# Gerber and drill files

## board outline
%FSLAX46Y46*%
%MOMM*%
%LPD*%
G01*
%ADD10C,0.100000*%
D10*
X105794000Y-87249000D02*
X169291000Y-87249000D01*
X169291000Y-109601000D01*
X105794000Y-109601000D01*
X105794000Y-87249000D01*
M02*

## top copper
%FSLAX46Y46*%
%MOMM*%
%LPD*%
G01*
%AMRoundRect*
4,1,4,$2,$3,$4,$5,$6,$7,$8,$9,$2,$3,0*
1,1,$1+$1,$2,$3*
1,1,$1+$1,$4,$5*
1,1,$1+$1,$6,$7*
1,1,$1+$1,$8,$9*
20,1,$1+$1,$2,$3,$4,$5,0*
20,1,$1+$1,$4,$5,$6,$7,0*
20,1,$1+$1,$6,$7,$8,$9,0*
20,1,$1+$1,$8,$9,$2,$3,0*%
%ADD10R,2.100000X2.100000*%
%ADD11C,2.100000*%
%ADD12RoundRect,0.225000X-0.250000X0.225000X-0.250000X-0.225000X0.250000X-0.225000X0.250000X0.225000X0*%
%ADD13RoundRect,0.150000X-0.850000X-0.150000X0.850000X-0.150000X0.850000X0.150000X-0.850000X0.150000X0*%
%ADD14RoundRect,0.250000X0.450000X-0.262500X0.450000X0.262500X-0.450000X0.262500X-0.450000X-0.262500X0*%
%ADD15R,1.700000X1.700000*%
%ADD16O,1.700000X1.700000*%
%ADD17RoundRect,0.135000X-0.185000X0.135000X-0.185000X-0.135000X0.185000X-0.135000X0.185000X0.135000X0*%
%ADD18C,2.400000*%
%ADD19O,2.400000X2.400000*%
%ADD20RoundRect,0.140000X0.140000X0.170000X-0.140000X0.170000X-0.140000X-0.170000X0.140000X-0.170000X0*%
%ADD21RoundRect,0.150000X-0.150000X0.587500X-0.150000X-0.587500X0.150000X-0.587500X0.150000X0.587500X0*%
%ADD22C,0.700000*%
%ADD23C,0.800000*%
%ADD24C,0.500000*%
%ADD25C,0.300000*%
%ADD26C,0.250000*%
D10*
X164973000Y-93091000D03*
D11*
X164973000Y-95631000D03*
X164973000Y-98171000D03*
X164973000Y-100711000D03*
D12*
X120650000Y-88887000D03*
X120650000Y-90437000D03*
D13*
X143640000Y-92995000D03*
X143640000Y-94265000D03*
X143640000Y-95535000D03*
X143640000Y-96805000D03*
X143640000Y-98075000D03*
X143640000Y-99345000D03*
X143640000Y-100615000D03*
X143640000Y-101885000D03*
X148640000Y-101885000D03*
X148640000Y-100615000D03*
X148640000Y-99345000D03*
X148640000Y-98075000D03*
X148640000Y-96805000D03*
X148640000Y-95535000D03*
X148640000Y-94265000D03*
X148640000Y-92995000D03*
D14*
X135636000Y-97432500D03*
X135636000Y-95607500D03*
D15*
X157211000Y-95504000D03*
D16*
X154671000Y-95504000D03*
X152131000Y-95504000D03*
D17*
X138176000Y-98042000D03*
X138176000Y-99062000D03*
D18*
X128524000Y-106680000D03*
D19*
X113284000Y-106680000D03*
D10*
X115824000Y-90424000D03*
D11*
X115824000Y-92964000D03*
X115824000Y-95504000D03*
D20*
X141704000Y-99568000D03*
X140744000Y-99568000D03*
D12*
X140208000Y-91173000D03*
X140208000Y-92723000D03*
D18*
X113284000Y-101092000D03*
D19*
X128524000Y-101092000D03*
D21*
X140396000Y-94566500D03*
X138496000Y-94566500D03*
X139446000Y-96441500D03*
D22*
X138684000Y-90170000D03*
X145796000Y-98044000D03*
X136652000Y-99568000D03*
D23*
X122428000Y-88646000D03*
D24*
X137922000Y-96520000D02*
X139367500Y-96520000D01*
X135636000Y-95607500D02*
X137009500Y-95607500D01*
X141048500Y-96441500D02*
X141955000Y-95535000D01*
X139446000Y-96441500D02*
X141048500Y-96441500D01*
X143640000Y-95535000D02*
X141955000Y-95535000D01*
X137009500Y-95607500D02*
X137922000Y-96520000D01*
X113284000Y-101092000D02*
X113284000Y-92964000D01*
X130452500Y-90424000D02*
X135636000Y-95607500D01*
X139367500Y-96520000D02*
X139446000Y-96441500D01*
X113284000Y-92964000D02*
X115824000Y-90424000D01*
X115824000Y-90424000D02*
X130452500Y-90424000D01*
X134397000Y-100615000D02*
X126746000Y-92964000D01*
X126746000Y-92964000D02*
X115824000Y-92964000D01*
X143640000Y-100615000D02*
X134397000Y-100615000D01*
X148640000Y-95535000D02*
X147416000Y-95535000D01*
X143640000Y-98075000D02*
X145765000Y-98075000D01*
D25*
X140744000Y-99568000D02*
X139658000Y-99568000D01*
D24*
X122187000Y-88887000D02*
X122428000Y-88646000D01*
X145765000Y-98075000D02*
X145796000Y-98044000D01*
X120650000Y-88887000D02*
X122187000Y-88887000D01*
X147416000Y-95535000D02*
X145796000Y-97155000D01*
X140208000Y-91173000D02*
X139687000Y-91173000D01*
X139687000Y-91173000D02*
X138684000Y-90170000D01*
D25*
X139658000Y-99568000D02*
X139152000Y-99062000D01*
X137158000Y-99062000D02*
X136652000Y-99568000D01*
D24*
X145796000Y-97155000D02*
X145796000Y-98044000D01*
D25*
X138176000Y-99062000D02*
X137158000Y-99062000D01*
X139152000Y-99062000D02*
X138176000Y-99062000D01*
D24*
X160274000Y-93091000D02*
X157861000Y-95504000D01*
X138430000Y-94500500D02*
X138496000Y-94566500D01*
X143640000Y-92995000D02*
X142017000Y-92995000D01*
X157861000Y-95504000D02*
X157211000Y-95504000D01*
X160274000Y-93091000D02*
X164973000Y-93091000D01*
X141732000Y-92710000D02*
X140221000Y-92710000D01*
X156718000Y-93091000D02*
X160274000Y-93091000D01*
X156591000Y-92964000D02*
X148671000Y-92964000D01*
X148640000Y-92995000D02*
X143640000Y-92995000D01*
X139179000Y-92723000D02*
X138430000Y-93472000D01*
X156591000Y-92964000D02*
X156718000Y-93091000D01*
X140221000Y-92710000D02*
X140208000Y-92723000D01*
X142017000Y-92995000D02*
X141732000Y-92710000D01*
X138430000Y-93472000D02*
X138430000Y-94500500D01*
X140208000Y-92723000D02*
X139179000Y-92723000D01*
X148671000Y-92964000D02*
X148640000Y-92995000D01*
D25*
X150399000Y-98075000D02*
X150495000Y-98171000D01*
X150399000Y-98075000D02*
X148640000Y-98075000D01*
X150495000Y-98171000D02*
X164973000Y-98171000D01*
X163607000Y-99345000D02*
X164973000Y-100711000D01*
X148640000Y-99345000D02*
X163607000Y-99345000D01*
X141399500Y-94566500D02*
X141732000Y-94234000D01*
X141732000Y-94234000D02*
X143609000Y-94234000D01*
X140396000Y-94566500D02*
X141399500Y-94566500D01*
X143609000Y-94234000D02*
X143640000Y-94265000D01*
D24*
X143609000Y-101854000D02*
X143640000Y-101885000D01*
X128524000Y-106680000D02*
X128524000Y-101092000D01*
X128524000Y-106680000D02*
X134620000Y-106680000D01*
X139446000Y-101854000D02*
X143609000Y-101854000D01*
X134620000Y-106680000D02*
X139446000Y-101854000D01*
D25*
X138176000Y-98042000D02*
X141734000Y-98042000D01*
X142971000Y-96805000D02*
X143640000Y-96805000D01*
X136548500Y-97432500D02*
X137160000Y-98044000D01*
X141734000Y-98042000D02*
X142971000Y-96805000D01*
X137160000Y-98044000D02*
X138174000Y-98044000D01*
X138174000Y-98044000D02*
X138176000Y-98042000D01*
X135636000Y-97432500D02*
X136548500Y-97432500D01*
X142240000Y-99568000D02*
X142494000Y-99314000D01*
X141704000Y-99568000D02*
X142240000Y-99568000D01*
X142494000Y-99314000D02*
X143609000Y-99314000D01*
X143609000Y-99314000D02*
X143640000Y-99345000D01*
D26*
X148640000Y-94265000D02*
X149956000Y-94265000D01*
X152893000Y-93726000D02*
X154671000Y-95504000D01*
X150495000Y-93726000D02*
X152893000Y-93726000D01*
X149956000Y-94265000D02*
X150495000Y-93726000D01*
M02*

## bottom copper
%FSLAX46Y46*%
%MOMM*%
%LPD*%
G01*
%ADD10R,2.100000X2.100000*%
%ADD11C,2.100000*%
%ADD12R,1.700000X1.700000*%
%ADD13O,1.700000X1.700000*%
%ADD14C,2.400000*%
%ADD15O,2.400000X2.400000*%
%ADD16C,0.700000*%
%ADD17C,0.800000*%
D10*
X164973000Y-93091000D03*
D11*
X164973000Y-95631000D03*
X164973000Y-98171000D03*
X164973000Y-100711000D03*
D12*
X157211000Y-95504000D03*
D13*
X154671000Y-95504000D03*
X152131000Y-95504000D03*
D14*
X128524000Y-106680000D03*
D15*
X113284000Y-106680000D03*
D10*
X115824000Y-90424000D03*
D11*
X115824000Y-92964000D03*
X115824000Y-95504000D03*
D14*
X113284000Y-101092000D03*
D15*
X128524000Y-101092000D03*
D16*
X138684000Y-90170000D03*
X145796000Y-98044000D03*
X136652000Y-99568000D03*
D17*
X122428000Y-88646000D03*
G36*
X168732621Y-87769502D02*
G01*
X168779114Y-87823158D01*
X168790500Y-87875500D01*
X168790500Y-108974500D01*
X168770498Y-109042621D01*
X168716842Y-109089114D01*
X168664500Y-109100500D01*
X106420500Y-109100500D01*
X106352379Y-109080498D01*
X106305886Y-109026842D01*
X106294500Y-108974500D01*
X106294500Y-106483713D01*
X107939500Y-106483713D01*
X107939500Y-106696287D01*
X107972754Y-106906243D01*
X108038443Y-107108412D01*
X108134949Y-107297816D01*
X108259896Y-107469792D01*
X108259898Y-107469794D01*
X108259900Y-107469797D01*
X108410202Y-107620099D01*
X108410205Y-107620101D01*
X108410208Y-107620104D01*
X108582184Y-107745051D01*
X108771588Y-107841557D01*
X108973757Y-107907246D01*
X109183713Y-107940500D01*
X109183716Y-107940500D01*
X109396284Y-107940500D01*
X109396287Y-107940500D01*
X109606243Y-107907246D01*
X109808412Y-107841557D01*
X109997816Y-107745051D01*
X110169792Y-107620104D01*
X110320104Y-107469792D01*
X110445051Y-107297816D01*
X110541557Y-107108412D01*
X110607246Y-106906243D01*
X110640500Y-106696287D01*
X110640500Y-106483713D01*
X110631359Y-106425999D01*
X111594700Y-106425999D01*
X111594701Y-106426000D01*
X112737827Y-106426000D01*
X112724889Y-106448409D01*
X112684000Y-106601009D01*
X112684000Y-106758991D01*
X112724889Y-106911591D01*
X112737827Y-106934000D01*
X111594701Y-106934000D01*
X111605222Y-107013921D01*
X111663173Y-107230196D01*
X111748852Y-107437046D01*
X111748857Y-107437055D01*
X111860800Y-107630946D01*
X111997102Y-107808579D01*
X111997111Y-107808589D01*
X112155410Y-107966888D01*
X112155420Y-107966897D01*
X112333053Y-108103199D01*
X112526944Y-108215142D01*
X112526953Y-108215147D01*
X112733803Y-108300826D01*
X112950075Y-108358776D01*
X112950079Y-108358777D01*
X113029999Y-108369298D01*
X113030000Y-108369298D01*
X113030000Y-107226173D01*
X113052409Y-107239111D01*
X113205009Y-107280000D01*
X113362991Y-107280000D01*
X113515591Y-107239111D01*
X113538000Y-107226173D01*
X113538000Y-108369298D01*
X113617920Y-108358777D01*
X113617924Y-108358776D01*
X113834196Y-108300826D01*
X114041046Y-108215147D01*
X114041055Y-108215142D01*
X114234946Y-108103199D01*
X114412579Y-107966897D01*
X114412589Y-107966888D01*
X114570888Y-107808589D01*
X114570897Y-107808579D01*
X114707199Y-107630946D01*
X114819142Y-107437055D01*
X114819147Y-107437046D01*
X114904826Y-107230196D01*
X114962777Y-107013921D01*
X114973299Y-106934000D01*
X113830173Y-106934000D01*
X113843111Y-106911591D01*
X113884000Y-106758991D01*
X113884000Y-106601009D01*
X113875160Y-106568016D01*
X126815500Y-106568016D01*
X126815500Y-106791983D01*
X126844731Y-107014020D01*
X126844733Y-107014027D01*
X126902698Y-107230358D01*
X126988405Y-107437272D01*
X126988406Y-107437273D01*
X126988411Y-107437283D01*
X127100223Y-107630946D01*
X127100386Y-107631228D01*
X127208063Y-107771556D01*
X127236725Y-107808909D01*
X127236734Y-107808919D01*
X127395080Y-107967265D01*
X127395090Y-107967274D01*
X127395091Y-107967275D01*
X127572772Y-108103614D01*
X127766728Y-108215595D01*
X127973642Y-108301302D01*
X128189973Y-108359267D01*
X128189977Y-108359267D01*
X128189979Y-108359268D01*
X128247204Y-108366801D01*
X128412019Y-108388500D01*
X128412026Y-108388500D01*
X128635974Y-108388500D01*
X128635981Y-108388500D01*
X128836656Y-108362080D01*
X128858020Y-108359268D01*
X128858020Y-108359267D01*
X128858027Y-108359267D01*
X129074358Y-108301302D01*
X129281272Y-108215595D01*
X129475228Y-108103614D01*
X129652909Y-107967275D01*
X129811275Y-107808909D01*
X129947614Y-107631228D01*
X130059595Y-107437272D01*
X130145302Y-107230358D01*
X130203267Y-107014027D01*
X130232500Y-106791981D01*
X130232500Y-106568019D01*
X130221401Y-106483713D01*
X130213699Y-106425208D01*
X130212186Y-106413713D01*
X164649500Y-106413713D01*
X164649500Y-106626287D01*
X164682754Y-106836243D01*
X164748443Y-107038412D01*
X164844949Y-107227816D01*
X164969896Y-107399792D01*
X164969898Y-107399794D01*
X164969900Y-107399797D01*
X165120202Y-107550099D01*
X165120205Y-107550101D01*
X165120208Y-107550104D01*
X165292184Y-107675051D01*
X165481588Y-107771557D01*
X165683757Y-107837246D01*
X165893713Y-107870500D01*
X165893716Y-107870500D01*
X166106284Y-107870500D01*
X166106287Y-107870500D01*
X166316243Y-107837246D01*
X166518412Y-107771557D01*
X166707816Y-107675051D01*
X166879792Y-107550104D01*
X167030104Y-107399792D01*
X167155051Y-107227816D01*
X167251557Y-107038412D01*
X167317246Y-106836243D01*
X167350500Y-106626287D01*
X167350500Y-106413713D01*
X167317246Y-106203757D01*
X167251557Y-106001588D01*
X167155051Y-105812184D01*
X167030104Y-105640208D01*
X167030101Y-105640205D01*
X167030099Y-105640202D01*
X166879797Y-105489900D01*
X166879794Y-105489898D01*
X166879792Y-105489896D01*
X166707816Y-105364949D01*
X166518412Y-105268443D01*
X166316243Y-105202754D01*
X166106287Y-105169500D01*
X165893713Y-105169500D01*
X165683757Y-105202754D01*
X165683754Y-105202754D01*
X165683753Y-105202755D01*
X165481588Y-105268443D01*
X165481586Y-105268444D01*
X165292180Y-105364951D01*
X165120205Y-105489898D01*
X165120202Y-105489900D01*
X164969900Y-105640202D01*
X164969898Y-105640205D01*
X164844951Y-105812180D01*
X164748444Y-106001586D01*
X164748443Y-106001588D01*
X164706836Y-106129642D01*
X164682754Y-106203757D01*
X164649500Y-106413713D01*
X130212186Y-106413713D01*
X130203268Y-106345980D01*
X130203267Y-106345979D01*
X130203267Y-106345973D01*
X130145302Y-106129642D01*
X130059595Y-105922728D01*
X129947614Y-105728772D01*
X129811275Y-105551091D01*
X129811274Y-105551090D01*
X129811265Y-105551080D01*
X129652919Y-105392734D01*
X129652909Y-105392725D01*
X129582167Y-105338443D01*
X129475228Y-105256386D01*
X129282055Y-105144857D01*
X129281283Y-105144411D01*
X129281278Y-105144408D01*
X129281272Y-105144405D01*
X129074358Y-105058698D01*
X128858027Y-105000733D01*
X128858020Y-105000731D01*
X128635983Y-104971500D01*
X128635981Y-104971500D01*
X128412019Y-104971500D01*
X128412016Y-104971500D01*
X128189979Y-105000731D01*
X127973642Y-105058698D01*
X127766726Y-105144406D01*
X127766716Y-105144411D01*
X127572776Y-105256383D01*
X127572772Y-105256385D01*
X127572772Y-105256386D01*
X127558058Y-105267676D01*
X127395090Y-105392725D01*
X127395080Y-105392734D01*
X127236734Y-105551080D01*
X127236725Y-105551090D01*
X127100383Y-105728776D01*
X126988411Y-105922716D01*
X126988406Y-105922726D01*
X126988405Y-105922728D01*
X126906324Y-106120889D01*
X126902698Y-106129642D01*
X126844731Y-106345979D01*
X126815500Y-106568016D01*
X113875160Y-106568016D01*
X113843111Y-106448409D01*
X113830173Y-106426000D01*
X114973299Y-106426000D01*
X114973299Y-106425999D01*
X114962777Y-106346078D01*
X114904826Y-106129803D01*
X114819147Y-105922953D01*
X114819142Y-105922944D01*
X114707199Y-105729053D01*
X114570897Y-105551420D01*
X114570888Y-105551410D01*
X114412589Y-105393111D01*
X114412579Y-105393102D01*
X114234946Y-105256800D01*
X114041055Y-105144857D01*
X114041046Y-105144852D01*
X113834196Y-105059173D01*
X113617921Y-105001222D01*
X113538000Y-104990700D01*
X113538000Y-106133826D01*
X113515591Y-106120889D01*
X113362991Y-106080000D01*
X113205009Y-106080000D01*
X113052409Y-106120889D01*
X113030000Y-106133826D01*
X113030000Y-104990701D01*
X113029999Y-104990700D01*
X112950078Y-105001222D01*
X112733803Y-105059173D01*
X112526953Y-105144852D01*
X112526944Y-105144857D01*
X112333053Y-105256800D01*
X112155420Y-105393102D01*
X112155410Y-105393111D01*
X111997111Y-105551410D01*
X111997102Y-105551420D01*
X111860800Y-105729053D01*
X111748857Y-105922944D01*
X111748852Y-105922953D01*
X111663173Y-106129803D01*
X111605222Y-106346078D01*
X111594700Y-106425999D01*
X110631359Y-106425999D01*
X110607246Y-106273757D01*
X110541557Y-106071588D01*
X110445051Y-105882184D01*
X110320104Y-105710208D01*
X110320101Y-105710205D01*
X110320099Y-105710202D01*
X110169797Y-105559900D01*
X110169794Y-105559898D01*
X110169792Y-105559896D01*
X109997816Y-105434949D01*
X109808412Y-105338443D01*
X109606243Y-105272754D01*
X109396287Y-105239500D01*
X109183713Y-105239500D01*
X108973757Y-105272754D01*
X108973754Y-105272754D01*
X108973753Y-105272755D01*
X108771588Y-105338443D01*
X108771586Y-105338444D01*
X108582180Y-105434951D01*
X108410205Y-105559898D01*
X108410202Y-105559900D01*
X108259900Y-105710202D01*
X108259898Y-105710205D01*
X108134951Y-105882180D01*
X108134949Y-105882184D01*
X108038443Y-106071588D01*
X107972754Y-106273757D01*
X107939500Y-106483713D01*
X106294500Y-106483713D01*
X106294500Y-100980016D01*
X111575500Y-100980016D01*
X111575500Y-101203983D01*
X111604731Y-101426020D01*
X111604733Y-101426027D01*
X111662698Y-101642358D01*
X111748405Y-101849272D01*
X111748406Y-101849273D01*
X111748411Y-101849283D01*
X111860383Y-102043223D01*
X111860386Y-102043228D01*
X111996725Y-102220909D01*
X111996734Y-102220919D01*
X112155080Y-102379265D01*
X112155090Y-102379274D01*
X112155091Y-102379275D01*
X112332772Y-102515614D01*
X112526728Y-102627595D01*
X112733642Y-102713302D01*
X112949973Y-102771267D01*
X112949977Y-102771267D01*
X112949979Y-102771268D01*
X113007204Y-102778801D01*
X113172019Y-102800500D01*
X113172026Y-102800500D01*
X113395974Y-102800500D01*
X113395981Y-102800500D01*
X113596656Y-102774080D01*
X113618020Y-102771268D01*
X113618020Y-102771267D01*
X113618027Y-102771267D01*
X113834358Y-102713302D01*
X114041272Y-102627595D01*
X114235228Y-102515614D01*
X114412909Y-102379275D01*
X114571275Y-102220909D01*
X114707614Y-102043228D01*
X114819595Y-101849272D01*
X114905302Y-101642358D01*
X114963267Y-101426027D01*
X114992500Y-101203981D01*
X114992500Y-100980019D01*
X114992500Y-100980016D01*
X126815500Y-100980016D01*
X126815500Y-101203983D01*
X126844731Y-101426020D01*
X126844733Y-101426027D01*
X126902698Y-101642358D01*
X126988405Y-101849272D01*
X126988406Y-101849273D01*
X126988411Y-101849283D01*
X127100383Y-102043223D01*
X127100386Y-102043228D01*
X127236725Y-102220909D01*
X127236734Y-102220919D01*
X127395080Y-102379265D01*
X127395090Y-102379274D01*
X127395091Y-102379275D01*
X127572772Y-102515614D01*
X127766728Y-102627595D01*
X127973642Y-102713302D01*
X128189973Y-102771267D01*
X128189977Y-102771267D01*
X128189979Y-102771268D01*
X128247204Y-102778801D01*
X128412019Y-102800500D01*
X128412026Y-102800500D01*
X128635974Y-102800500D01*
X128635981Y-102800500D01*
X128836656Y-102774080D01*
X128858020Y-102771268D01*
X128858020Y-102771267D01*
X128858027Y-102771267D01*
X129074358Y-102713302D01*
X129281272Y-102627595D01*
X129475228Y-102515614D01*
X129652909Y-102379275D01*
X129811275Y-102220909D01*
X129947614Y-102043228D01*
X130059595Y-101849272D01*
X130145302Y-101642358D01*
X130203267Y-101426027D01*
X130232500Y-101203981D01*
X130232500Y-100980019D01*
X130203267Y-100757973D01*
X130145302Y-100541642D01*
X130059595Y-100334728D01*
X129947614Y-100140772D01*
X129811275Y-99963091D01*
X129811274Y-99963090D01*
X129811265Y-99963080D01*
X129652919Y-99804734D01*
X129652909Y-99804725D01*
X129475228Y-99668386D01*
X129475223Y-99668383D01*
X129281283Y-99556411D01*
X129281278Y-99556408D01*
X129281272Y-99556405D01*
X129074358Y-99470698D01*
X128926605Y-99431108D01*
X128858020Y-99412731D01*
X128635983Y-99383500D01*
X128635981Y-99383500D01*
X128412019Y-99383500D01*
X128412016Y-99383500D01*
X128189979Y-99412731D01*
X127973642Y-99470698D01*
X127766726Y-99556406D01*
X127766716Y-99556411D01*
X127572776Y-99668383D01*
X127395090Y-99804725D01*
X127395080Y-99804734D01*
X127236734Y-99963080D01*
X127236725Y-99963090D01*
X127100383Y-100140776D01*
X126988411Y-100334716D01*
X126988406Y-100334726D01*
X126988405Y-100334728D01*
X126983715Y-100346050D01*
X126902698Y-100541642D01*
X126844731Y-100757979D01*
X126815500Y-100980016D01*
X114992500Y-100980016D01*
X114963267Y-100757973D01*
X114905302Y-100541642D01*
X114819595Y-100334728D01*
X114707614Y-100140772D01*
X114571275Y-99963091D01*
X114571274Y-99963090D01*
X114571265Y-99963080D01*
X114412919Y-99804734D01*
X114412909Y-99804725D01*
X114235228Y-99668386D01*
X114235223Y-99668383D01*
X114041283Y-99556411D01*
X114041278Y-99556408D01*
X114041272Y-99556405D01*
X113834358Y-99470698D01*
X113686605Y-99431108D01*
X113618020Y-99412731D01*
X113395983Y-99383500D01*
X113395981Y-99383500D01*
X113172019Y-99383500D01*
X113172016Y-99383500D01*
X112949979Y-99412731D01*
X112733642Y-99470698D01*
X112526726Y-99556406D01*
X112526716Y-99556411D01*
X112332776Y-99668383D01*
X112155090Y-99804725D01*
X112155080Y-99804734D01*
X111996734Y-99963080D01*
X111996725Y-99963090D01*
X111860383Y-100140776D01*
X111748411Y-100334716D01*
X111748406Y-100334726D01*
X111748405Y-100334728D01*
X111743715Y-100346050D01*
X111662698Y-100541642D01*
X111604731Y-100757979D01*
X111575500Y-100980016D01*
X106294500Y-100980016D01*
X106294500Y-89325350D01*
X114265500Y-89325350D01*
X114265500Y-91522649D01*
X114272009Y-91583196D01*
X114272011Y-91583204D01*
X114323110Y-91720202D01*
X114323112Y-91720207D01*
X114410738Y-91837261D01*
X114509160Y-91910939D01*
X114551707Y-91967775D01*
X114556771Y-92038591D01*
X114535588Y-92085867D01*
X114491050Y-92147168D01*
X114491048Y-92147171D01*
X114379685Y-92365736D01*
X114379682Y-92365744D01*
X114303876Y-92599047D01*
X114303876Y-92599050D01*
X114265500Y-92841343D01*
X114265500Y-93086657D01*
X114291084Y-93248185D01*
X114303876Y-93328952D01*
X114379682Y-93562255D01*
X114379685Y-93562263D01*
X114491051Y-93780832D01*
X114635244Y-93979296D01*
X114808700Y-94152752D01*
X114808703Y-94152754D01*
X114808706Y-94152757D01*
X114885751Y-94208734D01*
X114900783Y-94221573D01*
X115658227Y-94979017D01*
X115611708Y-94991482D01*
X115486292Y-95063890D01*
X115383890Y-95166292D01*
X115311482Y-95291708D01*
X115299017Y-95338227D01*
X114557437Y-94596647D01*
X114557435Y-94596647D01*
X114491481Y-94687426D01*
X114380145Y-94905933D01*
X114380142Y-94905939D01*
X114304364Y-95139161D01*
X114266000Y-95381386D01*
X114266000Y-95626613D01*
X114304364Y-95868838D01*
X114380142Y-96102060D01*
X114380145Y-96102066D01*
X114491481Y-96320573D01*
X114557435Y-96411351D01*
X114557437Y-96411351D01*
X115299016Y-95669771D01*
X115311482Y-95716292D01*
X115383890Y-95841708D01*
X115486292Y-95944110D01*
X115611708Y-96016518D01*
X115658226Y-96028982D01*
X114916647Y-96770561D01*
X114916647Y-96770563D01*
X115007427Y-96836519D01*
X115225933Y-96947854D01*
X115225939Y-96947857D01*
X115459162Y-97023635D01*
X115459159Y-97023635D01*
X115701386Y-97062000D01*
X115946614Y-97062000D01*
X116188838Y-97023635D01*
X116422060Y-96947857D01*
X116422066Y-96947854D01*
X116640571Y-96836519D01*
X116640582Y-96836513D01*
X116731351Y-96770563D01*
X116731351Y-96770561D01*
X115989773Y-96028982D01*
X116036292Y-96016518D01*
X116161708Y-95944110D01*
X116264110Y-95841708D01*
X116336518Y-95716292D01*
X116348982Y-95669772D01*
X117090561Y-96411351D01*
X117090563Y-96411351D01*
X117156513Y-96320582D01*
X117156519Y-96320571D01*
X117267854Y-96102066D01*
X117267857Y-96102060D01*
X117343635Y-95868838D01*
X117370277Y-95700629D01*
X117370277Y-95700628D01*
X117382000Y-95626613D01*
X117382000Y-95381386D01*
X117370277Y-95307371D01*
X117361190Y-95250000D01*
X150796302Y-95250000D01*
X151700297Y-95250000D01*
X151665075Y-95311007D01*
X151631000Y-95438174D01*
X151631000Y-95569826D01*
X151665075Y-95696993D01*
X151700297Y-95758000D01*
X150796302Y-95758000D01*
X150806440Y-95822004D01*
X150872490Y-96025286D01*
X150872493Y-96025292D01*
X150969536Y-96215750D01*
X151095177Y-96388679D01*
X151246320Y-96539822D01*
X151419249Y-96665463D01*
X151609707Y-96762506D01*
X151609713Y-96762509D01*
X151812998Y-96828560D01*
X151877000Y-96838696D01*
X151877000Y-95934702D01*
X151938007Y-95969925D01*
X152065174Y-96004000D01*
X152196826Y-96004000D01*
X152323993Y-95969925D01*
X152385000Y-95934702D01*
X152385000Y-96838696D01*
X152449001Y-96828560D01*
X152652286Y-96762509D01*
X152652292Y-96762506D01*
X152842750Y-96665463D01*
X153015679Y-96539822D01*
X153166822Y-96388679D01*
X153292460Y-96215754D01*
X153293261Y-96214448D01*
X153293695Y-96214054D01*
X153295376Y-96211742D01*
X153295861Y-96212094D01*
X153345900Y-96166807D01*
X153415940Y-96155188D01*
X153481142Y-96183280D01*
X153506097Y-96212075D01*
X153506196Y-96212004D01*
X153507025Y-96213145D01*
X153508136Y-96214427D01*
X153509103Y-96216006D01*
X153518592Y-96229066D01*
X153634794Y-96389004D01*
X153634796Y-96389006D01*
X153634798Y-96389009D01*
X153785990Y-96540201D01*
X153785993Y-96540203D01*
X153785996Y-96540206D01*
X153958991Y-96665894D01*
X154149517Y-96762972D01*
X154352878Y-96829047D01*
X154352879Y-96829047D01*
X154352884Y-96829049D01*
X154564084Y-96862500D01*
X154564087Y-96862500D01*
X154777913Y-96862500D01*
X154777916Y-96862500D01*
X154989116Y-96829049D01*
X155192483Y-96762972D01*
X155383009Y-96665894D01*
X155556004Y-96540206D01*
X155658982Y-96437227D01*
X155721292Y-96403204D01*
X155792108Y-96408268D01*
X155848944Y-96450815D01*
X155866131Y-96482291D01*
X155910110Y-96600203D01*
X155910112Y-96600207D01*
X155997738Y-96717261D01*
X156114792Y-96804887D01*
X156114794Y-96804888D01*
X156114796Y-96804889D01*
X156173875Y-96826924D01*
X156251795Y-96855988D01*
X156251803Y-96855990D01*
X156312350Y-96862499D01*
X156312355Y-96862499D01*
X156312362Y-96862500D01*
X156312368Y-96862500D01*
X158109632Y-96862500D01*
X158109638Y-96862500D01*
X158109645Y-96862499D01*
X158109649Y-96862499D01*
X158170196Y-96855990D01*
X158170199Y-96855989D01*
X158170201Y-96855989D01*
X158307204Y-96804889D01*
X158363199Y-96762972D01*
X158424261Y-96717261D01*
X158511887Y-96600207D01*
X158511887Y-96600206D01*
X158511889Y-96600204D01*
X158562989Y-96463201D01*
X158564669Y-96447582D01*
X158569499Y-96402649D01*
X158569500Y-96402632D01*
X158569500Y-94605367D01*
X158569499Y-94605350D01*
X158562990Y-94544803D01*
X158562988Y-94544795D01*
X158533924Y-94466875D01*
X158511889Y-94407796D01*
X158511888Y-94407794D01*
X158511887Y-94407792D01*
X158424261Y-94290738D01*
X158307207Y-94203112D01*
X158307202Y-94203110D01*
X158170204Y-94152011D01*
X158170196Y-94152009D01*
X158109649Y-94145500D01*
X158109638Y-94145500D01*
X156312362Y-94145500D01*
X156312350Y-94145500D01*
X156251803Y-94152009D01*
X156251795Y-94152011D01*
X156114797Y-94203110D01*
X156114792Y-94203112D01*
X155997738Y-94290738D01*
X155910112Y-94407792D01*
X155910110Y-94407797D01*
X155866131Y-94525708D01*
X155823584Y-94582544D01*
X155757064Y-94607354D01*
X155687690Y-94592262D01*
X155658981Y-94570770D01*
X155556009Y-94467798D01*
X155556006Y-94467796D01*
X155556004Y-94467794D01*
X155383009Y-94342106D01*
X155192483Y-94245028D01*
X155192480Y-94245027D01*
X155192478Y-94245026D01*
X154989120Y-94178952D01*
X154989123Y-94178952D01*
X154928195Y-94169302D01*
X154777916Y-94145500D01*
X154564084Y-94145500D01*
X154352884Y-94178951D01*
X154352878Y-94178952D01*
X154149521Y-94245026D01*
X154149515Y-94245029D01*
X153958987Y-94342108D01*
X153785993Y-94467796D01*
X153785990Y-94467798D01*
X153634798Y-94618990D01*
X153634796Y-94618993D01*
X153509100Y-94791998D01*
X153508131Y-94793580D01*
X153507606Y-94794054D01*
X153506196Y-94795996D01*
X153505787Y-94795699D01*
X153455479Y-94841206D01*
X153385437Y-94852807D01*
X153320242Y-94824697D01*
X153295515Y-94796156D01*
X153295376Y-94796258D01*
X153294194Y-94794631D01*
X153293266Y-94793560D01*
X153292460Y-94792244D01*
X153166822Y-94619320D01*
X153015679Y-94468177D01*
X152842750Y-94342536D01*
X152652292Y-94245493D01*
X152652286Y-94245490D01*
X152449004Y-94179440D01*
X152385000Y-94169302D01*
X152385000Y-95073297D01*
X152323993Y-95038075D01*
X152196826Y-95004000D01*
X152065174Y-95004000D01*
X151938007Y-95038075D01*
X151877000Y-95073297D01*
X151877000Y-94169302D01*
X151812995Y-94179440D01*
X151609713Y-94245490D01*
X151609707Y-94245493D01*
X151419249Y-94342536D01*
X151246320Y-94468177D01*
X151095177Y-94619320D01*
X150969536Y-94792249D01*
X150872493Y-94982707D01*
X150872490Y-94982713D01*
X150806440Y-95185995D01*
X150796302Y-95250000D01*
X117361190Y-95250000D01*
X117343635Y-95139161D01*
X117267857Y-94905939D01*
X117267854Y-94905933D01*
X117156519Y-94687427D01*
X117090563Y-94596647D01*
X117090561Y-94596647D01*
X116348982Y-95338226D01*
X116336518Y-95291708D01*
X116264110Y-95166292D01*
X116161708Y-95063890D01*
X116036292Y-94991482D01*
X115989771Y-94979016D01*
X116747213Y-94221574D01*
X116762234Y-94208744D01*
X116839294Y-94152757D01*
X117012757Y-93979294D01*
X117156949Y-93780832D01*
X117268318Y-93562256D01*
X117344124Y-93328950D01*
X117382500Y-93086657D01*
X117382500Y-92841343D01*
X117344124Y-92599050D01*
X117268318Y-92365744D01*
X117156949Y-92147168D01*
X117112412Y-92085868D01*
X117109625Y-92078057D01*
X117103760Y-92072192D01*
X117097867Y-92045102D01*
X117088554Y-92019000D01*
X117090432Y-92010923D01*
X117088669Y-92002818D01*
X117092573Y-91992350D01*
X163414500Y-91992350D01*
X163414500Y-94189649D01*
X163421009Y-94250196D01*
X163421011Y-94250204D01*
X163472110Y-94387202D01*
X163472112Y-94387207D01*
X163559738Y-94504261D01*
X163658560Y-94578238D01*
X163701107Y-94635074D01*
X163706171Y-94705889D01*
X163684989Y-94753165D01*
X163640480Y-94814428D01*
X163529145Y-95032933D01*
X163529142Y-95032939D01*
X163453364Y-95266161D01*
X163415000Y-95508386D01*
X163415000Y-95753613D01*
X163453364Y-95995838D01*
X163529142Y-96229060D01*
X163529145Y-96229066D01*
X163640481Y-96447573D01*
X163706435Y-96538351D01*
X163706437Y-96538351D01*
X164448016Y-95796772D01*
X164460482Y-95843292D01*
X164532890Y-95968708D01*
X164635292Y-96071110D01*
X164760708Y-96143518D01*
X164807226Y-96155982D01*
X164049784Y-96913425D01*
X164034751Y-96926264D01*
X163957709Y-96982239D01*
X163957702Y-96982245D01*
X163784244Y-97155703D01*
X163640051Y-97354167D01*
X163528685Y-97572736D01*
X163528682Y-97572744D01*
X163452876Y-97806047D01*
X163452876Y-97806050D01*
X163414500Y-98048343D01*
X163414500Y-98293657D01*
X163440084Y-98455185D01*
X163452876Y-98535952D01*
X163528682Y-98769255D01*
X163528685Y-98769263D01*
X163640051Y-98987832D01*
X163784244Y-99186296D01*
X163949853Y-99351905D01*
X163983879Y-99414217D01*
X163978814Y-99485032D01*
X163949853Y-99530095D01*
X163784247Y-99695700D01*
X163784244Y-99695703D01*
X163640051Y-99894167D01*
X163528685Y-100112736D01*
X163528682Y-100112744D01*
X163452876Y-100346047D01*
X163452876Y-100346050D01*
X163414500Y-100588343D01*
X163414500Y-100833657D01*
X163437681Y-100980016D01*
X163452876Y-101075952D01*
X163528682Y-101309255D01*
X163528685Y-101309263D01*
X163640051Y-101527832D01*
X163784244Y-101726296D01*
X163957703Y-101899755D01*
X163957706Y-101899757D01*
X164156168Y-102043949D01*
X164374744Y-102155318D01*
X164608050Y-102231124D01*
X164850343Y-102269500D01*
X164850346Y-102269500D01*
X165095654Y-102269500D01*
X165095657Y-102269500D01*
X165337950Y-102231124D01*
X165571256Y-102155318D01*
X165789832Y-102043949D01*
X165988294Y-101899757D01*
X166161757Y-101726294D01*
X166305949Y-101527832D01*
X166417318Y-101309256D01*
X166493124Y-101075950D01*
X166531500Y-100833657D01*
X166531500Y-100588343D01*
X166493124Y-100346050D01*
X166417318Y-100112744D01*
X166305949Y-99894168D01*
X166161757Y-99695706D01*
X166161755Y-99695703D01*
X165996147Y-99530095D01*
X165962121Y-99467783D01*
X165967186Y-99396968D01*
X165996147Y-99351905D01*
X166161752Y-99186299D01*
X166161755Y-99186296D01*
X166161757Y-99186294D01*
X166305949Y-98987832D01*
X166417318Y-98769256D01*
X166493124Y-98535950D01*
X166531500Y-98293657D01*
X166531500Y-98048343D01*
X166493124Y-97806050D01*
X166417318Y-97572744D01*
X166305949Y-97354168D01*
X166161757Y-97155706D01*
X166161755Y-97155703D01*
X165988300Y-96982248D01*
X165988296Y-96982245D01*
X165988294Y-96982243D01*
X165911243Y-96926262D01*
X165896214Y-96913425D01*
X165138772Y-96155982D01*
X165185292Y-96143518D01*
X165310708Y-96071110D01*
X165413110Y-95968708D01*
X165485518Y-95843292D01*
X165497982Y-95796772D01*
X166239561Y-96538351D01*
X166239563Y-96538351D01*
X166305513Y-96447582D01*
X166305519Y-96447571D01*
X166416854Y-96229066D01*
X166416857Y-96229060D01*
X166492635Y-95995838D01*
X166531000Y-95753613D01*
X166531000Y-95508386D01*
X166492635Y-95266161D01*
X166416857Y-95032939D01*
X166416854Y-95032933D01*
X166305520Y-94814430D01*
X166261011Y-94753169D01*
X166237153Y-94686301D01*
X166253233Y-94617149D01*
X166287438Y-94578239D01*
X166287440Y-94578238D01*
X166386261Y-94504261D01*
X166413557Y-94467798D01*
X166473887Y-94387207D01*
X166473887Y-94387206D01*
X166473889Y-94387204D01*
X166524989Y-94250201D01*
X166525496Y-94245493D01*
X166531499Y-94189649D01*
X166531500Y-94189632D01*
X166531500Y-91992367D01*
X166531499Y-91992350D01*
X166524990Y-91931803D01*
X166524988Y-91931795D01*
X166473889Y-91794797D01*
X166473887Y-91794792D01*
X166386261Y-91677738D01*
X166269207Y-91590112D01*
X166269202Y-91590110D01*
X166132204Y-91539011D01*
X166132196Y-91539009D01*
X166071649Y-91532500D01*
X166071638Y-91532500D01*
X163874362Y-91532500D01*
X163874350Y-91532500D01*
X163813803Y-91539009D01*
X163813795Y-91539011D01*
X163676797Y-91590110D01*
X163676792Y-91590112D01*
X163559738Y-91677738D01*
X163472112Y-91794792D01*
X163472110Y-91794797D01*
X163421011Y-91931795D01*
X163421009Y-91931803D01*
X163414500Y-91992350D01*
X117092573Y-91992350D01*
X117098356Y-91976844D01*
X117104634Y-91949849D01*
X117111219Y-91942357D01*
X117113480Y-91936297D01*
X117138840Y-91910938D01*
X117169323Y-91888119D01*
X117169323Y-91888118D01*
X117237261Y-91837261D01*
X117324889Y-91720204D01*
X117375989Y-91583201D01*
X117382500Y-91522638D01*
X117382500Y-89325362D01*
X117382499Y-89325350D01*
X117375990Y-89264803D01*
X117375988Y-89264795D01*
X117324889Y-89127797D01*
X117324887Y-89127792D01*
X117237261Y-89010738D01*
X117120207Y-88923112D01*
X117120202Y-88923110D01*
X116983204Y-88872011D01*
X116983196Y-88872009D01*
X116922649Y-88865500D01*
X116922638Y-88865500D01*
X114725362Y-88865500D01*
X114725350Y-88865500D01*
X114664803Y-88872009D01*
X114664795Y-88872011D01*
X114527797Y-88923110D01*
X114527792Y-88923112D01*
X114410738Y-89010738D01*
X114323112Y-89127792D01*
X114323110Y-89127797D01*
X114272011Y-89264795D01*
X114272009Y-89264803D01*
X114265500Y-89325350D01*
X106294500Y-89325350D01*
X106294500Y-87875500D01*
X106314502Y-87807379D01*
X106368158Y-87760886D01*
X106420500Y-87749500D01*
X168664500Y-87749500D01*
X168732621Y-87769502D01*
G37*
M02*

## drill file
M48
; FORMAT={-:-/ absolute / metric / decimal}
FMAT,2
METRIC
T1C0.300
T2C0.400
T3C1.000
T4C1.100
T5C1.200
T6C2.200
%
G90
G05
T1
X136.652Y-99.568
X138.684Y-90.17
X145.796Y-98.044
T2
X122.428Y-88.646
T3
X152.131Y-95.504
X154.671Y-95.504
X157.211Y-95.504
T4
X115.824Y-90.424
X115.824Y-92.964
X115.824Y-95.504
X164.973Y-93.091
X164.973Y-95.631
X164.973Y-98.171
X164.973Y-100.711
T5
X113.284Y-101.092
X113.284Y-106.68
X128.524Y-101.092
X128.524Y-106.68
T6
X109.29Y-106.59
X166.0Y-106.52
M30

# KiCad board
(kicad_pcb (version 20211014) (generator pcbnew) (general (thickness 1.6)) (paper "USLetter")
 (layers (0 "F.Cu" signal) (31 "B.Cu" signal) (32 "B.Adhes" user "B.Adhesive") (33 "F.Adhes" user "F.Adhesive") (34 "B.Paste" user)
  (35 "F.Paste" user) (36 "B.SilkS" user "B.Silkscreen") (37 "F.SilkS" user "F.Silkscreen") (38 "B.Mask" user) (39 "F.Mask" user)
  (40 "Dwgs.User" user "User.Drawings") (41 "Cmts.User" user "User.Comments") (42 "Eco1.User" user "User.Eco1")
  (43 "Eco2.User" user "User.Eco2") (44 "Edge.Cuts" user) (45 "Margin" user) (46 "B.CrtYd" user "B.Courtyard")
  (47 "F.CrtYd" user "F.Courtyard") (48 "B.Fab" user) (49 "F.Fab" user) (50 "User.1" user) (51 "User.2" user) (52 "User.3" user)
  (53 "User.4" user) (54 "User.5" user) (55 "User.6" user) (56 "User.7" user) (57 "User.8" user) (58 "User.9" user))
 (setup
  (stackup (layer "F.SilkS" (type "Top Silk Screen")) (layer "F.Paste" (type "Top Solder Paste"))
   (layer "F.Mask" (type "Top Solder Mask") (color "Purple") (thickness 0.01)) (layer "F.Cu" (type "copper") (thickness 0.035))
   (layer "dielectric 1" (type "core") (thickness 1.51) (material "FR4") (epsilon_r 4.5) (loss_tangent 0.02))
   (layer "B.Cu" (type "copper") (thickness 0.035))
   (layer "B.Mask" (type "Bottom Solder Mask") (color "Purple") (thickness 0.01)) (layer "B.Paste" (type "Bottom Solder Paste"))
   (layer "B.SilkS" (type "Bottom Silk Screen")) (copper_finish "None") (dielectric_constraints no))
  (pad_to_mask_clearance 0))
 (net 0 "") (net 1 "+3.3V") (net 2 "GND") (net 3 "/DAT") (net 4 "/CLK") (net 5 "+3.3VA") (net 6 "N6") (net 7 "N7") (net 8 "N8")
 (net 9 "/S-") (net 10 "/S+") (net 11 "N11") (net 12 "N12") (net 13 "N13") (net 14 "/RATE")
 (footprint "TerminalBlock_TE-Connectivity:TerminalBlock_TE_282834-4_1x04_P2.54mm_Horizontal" (layer "F.Cu") (at 164.973 93.091 -90)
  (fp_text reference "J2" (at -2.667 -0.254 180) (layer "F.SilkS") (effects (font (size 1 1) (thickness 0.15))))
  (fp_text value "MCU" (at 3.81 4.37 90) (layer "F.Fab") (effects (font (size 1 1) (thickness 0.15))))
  (pad "1" thru_hole rect (at 0 0 270) (size 2.1 2.1) (drill 1.1) (layers *.Cu *.Mask) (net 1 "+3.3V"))
  (pad "2" thru_hole circle (at 2.54 0 270) (size 2.1 2.1) (drill 1.1) (layers *.Cu *.Mask) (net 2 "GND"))
  (pad "3" thru_hole circle (at 5.08 0 270) (size 2.1 2.1) (drill 1.1) (layers *.Cu *.Mask) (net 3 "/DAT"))
  (pad "4" thru_hole circle (at 7.62 0 270) (size 2.1 2.1) (drill 1.1) (layers *.Cu *.Mask) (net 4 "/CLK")))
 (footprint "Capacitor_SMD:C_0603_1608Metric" (layer "F.Cu") (at 120.65 89.662 -90)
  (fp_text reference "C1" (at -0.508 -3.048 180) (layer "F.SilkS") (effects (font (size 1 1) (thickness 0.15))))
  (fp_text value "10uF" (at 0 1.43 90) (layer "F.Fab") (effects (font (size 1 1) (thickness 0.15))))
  (pad "1" smd roundrect (at -0.775 0 270) (size 0.9 0.95) (layers "F.Cu" "F.Paste" "F.Mask") (roundrect_rratio 0.25) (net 2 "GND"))
  (pad "2" smd roundrect (at 0.775 0 270) (size 0.9 0.95) (layers "F.Cu" "F.Paste" "F.Mask") (roundrect_rratio 0.25) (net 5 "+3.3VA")))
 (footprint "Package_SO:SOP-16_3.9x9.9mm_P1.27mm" (layer "F.Cu") (at 146.14 97.44)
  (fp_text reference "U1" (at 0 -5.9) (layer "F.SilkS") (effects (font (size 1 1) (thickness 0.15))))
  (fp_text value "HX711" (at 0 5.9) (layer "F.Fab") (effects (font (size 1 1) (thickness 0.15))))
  (pad "1" smd roundrect (at -2.5 -4.445) (size 2 0.6) (layers "F.Cu" "F.Paste" "F.Mask") (roundrect_rratio 0.25) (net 1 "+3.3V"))
  (pad "2" smd roundrect (at -2.5 -3.175) (size 2 0.6) (layers "F.Cu" "F.Paste" "F.Mask") (roundrect_rratio 0.25) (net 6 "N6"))
  (pad "3" smd roundrect (at -2.5 -1.905) (size 2 0.6) (layers "F.Cu" "F.Paste" "F.Mask") (roundrect_rratio 0.25) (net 5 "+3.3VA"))
  (pad "4" smd roundrect (at -2.5 -0.635) (size 2 0.6) (layers "F.Cu" "F.Paste" "F.Mask") (roundrect_rratio 0.25) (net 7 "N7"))
  (pad "5" smd roundrect (at -2.5 0.635) (size 2 0.6) (layers "F.Cu" "F.Paste" "F.Mask") (roundrect_rratio 0.25) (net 2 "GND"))
  (pad "6" smd roundrect (at -2.5 1.905) (size 2 0.6) (layers "F.Cu" "F.Paste" "F.Mask") (roundrect_rratio 0.25) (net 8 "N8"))
  (pad "7" smd roundrect (at -2.5 3.175) (size 2 0.6) (layers "F.Cu" "F.Paste" "F.Mask") (roundrect_rratio 0.25) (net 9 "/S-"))
  (pad "8" smd roundrect (at -2.5 4.445) (size 2 0.6) (layers "F.Cu" "F.Paste" "F.Mask") (roundrect_rratio 0.25) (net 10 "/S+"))
  (pad "9" smd roundrect (at 2.5 4.445) (size 2 0.6) (layers "F.Cu" "F.Paste" "F.Mask") (roundrect_rratio 0.25) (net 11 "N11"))
  (pad "10" smd roundrect (at 2.5 3.175) (size 2 0.6) (layers "F.Cu" "F.Paste" "F.Mask") (roundrect_rratio 0.25) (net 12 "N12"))
  (pad "11" smd roundrect (at 2.5 1.905) (size 2 0.6) (layers "F.Cu" "F.Paste" "F.Mask") (roundrect_rratio 0.25) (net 4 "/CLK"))
  (pad "12" smd roundrect (at 2.5 0.635) (size 2 0.6) (layers "F.Cu" "F.Paste" "F.Mask") (roundrect_rratio 0.25) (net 3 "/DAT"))
  (pad "13" smd roundrect (at 2.5 -0.635) (size 2 0.6) (layers "F.Cu" "F.Paste" "F.Mask") (roundrect_rratio 0.25) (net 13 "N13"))
  (pad "14" smd roundrect (at 2.5 -1.905) (size 2 0.6) (layers "F.Cu" "F.Paste" "F.Mask") (roundrect_rratio 0.25) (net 2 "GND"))
  (pad "15" smd roundrect (at 2.5 -3.175) (size 2 0.6) (layers "F.Cu" "F.Paste" "F.Mask") (roundrect_rratio 0.25) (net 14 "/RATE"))
  (pad "16" smd roundrect (at 2.5 -4.445) (size 2 0.6) (layers "F.Cu" "F.Paste" "F.Mask") (roundrect_rratio 0.25) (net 1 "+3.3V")))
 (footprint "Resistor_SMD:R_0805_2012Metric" (layer "F.Cu") (at 135.636 96.52 90)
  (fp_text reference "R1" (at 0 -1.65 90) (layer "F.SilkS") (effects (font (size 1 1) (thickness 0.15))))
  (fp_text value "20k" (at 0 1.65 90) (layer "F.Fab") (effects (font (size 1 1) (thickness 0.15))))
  (pad "1" smd roundrect (at -0.9125 0 90) (size 1.025 1.4) (layers "F.Cu" "F.Paste" "F.Mask") (roundrect_rratio 0.243902439) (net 7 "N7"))
  (pad "2" smd roundrect (at 0.9125 0 90) (size 1.025 1.4) (layers "F.Cu" "F.Paste" "F.Mask") (roundrect_rratio 0.243902439)
   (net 5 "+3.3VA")))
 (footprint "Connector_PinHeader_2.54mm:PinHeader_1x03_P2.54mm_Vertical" (layer "F.Cu") (at 157.211 95.504 -90)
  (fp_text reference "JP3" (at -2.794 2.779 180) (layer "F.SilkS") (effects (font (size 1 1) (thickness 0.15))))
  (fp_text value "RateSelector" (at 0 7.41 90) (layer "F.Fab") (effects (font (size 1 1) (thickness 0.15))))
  (pad "1" thru_hole rect (at 0 0 270) (size 1.7 1.7) (drill 1) (layers *.Cu *.Mask) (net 1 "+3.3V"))
  (pad "2" thru_hole oval (at 0 2.54 270) (size 1.7 1.7) (drill 1) (layers *.Cu *.Mask) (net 14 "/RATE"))
  (pad "3" thru_hole oval (at 0 5.08 270) (size 1.7 1.7) (drill 1) (layers *.Cu *.Mask) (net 2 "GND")))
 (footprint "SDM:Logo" (layer "F.Cu") (at 135.255 105.029)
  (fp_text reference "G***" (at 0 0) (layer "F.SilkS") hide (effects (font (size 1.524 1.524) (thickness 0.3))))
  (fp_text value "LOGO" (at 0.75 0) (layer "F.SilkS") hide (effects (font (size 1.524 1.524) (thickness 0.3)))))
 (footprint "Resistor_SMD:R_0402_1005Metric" (layer "F.Cu") (at 138.176 98.552 -90)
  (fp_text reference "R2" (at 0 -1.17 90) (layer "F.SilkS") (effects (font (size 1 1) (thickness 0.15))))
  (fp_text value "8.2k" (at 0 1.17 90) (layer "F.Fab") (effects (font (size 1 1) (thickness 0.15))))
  (pad "1" smd roundrect (at -0.51 0 270) (size 0.54 0.64) (layers "F.Cu" "F.Paste" "F.Mask") (roundrect_rratio 0.25) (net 7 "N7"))
  (pad "2" smd roundrect (at 0.51 0 270) (size 0.54 0.64) (layers "F.Cu" "F.Paste" "F.Mask") (roundrect_rratio 0.25) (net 2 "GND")))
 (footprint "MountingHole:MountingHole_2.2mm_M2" (layer "F.Cu") (at 109.29 106.59)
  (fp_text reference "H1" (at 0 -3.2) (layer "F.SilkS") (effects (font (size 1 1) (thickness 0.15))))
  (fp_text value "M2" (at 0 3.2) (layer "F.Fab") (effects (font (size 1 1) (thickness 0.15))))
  (pad "" np_thru_hole circle (at 0 0) (size 2.2 2.2) (drill 2.2) (layers *.Cu *.Mask)))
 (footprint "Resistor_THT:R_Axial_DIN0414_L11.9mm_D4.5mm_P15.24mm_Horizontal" (layer "F.Cu") (at 128.524 106.68 180)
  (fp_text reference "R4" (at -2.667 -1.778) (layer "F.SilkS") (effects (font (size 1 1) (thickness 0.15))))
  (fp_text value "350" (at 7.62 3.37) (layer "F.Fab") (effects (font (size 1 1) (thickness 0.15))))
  (pad "1" thru_hole circle (at 0 0 180) (size 2.4 2.4) (drill 1.2) (layers *.Cu *.Mask) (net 10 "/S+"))
  (pad "2" thru_hole oval (at 15.24 0 180) (size 2.4 2.4) (drill 1.2) (layers *.Cu *.Mask) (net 2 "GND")))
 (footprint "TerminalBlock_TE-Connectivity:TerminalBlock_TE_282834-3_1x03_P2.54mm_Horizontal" (layer "F.Cu") (at 115.824 90.424 -90)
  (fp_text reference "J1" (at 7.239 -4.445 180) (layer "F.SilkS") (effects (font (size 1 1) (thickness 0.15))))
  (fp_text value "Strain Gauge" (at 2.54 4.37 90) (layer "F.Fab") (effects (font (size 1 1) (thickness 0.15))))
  (pad "1" thru_hole rect (at 0 0 270) (size 2.1 2.1) (drill 1.1) (layers *.Cu *.Mask) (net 5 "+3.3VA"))
  (pad "2" thru_hole circle (at 2.54 0 270) (size 2.1 2.1) (drill 1.1) (layers *.Cu *.Mask) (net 9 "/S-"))
  (pad "3" thru_hole circle (at 5.08 0 270) (size 2.1 2.1) (drill 1.1) (layers *.Cu *.Mask) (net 2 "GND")))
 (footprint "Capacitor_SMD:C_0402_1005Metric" (layer "F.Cu") (at 141.224 99.568 180)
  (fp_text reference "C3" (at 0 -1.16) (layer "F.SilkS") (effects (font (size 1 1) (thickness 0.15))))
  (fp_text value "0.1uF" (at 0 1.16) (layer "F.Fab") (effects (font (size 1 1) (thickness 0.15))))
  (pad "1" smd roundrect (at -0.48 0 180) (size 0.56 0.62) (layers "F.Cu" "F.Paste" "F.Mask") (roundrect_rratio 0.25) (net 8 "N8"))
  (pad "2" smd roundrect (at 0.48 0 180) (size 0.56 0.62) (layers "F.Cu" "F.Paste" "F.Mask") (roundrect_rratio 0.25) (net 2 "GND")))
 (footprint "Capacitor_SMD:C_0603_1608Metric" (layer "F.Cu") (at 140.208 91.948 -90)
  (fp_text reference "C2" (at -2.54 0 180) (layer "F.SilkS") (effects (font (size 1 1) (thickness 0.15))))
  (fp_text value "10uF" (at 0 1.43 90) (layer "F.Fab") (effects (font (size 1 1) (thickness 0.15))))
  (pad "1" smd roundrect (at -0.775 0 270) (size 0.9 0.95) (layers "F.Cu" "F.Paste" "F.Mask") (roundrect_rratio 0.25) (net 2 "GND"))
  (pad "2" smd roundrect (at 0.775 0 270) (size 0.9 0.95) (layers "F.Cu" "F.Paste" "F.Mask") (roundrect_rratio 0.25) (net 1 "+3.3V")))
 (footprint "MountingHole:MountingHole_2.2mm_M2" (layer "F.Cu") (at 166 106.52)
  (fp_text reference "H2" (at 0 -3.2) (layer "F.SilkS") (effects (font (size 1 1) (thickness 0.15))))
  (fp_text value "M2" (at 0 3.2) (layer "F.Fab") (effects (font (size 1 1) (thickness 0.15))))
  (pad "" np_thru_hole circle (at 0 0) (size 2.2 2.2) (drill 2.2) (layers *.Cu *.Mask)))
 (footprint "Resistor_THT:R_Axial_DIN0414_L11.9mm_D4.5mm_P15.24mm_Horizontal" (layer "F.Cu") (at 113.284 101.092)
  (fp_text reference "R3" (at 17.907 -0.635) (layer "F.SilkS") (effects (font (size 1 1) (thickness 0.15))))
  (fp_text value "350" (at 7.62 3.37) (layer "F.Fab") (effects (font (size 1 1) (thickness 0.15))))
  (pad "1" thru_hole circle (at 0 0) (size 2.4 2.4) (drill 1.2) (layers *.Cu *.Mask) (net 5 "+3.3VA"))
  (pad "2" thru_hole oval (at 15.24 0) (size 2.4 2.4) (drill 1.2) (layers *.Cu *.Mask) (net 10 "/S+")))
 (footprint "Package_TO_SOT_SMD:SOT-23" (layer "F.Cu") (at 139.446 95.504 -90)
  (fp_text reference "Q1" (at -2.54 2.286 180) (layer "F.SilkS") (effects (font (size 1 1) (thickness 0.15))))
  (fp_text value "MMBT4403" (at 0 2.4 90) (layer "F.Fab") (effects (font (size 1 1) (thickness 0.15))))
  (pad "1" smd roundrect (at -0.9375 -0.95 270) (size 1.475 0.6) (layers "F.Cu" "F.Paste" "F.Mask") (roundrect_rratio 0.25) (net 6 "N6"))
  (pad "2" smd roundrect (at -0.9375 0.95 270) (size 1.475 0.6) (layers "F.Cu" "F.Paste" "F.Mask") (roundrect_rratio 0.25) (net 1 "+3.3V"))
  (pad "3" smd roundrect (at 0.9375 0 270) (size 1.475 0.6) (layers "F.Cu" "F.Paste" "F.Mask") (roundrect_rratio 0.25) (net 5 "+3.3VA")))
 (gr_rect (start 105.794 87.249) (end 169.291 109.601) (layer "Edge.Cuts") (width 0.1) (fill none))
 (segment (start 137.922 96.52) (end 139.3675 96.52) (width 0.5) (layer "F.Cu") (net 5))
 (segment (start 135.636 95.6075) (end 137.0095 95.6075) (width 0.5) (layer "F.Cu") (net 5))
 (segment (start 141.0485 96.4415) (end 141.955 95.535) (width 0.5) (layer "F.Cu") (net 5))
 (segment (start 139.446 96.4415) (end 141.0485 96.4415) (width 0.5) (layer "F.Cu") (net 5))
 (segment (start 143.64 95.535) (end 141.955 95.535) (width 0.5) (layer "F.Cu") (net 5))
 (segment (start 137.0095 95.6075) (end 137.922 96.52) (width 0.5) (layer "F.Cu") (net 5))
 (segment (start 113.284 101.092) (end 113.284 92.964) (width 0.5) (layer "F.Cu") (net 5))
 (segment (start 130.4525 90.424) (end 135.636 95.6075) (width 0.5) (layer "F.Cu") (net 5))
 (segment (start 139.3675 96.52) (end 139.446 96.4415) (width 0.5) (layer "F.Cu") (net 5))
 (segment (start 113.284 92.964) (end 115.824 90.424) (width 0.5) (layer "F.Cu") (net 5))
 (segment (start 115.824 90.424) (end 130.4525 90.424) (width 0.5) (layer "F.Cu") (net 5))
 (segment (start 134.397 100.615) (end 126.746 92.964) (width 0.5) (layer "F.Cu") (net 9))
 (segment (start 126.746 92.964) (end 115.824 92.964) (width 0.5) (layer "F.Cu") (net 9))
 (segment (start 143.64 100.615) (end 134.397 100.615) (width 0.5) (layer "F.Cu") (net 9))
 (segment (start 148.64 95.535) (end 147.416 95.535) (width 0.5) (layer "F.Cu") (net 2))
 (segment (start 143.64 98.075) (end 145.765 98.075) (width 0.5) (layer "F.Cu") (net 2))
 (segment (start 140.744 99.568) (end 139.658 99.568) (width 0.3) (layer "F.Cu") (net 2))
 (segment (start 122.187 88.887) (end 122.428 88.646) (width 0.5) (layer "F.Cu") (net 2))
 (segment (start 145.765 98.075) (end 145.796 98.044) (width 0.5) (layer "F.Cu") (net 2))
 (segment (start 120.65 88.887) (end 122.187 88.887) (width 0.5) (layer "F.Cu") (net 2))
 (segment (start 147.416 95.535) (end 145.796 97.155) (width 0.5) (layer "F.Cu") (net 2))
 (segment (start 140.208 91.173) (end 139.687 91.173) (width 0.5) (layer "F.Cu") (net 2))
 (segment (start 139.687 91.173) (end 138.684 90.17) (width 0.5) (layer "F.Cu") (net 2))
 (segment (start 139.658 99.568) (end 139.152 99.062) (width 0.3) (layer "F.Cu") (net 2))
 (segment (start 137.158 99.062) (end 136.652 99.568) (width 0.3) (layer "F.Cu") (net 2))
 (segment (start 145.796 97.155) (end 145.796 98.044) (width 0.5) (layer "F.Cu") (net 2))
 (segment (start 138.176 99.062) (end 137.158 99.062) (width 0.3) (layer "F.Cu") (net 2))
 (segment (start 139.152 99.062) (end 138.176 99.062) (width 0.3) (layer "F.Cu") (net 2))
 (via (at 138.684 90.17) (size 0.7) (drill 0.3) (layers "F.Cu" "B.Cu") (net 2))
 (via (at 145.796 98.044) (size 0.7) (drill 0.3) (layers "F.Cu" "B.Cu") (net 2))
 (via (at 136.652 99.568) (size 0.7) (drill 0.3) (layers "F.Cu" "B.Cu") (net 2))
 (via (at 122.428 88.646) (size 0.8) (drill 0.4) (layers "F.Cu" "B.Cu") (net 2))
 (segment (start 160.274 93.091) (end 157.861 95.504) (width 0.5) (layer "F.Cu") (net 1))
 (segment (start 138.43 94.5005) (end 138.496 94.5665) (width 0.5) (layer "F.Cu") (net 1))
 (segment (start 143.64 92.995) (end 142.017 92.995) (width 0.5) (layer "F.Cu") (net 1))
 (segment (start 157.861 95.504) (end 157.211 95.504) (width 0.5) (layer "F.Cu") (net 1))
 (segment (start 160.274 93.091) (end 164.973 93.091) (width 0.5) (layer "F.Cu") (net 1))
 (segment (start 141.732 92.71) (end 140.221 92.71) (width 0.5) (layer "F.Cu") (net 1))
 (segment (start 156.718 93.091) (end 160.274 93.091) (width 0.5) (layer "F.Cu") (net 1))
 (segment (start 156.591 92.964) (end 148.671 92.964) (width 0.5) (layer "F.Cu") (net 1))
 (segment (start 148.64 92.995) (end 143.64 92.995) (width 0.5) (layer "F.Cu") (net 1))
 (segment (start 139.179 92.723) (end 138.43 93.472) (width 0.5) (layer "F.Cu") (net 1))
 (segment (start 156.591 92.964) (end 156.718 93.091) (width 0.5) (layer "F.Cu") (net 1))
 (segment (start 140.221 92.71) (end 140.208 92.723) (width 0.5) (layer "F.Cu") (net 1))
 (segment (start 142.017 92.995) (end 141.732 92.71) (width 0.5) (layer "F.Cu") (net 1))
 (segment (start 138.43 93.472) (end 138.43 94.5005) (width 0.5) (layer "F.Cu") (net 1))
 (segment (start 140.208 92.723) (end 139.179 92.723) (width 0.5) (layer "F.Cu") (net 1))
 (segment (start 148.671 92.964) (end 148.64 92.995) (width 0.5) (layer "F.Cu") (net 1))
 (segment (start 150.399 98.075) (end 150.495 98.171) (width 0.3) (layer "F.Cu") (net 3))
 (segment (start 150.399 98.075) (end 148.64 98.075) (width 0.3) (layer "F.Cu") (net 3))
 (segment (start 150.495 98.171) (end 164.973 98.171) (width 0.3) (layer "F.Cu") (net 3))
 (segment (start 163.607 99.345) (end 164.973 100.711) (width 0.3) (layer "F.Cu") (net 4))
 (segment (start 148.64 99.345) (end 163.607 99.345) (width 0.3) (layer "F.Cu") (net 4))
 (segment (start 141.3995 94.5665) (end 141.732 94.234) (width 0.3) (layer "F.Cu") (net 6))
 (segment (start 141.732 94.234) (end 143.609 94.234) (width 0.3) (layer "F.Cu") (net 6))
 (segment (start 140.396 94.5665) (end 141.3995 94.5665) (width 0.3) (layer "F.Cu") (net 6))
 (segment (start 143.609 94.234) (end 143.64 94.265) (width 0.3) (layer "F.Cu") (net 6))
 (segment (start 143.609 101.854) (end 143.64 101.885) (width 0.5) (layer "F.Cu") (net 10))
 (segment (start 128.524 106.68) (end 128.524 101.092) (width 0.5) (layer "F.Cu") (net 10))
 (segment (start 128.524 106.68) (end 134.62 106.68) (width 0.5) (layer "F.Cu") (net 10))
 (segment (start 139.446 101.854) (end 143.609 101.854) (width 0.5) (layer "F.Cu") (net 10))
 (segment (start 134.62 106.68) (end 139.446 101.854) (width 0.5) (layer "F.Cu") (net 10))
 (segment (start 138.176 98.042) (end 141.734 98.042) (width 0.3) (layer "F.Cu") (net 7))
 (segment (start 142.971 96.805) (end 143.64 96.805) (width 0.3) (layer "F.Cu") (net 7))
 (segment (start 136.5485 97.4325) (end 137.16 98.044) (width 0.3) (layer "F.Cu") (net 7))
 (segment (start 141.734 98.042) (end 142.971 96.805) (width 0.3) (layer "F.Cu") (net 7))
 (segment (start 137.16 98.044) (end 138.174 98.044) (width 0.3) (layer "F.Cu") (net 7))
 (segment (start 138.174 98.044) (end 138.176 98.042) (width 0.3) (layer "F.Cu") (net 7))
 (segment (start 135.636 97.4325) (end 136.5485 97.4325) (width 0.3) (layer "F.Cu") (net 7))
 (segment (start 142.24 99.568) (end 142.494 99.314) (width 0.3) (layer "F.Cu") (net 8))
 (segment (start 141.704 99.568) (end 142.24 99.568) (width 0.3) (layer "F.Cu") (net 8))
 (segment (start 142.494 99.314) (end 143.609 99.314) (width 0.3) (layer "F.Cu") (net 8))
 (segment (start 143.609 99.314) (end 143.64 99.345) (width 0.3) (layer "F.Cu") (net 8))
 (segment (start 148.64 94.265) (end 149.956 94.265) (width 0.25) (layer "F.Cu") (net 14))
 (segment (start 152.893 93.726) (end 154.671 95.504) (width 0.25) (layer "F.Cu") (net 14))
 (segment (start 150.495 93.726) (end 152.893 93.726) (width 0.25) (layer "F.Cu") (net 14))
 (segment (start 149.956 94.265) (end 150.495 93.726) (width 0.25) (layer "F.Cu") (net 14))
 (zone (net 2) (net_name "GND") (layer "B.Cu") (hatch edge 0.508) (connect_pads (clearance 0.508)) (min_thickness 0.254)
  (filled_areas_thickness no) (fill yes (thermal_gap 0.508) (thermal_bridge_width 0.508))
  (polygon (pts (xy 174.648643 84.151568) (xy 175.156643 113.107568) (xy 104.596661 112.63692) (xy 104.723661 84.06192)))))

